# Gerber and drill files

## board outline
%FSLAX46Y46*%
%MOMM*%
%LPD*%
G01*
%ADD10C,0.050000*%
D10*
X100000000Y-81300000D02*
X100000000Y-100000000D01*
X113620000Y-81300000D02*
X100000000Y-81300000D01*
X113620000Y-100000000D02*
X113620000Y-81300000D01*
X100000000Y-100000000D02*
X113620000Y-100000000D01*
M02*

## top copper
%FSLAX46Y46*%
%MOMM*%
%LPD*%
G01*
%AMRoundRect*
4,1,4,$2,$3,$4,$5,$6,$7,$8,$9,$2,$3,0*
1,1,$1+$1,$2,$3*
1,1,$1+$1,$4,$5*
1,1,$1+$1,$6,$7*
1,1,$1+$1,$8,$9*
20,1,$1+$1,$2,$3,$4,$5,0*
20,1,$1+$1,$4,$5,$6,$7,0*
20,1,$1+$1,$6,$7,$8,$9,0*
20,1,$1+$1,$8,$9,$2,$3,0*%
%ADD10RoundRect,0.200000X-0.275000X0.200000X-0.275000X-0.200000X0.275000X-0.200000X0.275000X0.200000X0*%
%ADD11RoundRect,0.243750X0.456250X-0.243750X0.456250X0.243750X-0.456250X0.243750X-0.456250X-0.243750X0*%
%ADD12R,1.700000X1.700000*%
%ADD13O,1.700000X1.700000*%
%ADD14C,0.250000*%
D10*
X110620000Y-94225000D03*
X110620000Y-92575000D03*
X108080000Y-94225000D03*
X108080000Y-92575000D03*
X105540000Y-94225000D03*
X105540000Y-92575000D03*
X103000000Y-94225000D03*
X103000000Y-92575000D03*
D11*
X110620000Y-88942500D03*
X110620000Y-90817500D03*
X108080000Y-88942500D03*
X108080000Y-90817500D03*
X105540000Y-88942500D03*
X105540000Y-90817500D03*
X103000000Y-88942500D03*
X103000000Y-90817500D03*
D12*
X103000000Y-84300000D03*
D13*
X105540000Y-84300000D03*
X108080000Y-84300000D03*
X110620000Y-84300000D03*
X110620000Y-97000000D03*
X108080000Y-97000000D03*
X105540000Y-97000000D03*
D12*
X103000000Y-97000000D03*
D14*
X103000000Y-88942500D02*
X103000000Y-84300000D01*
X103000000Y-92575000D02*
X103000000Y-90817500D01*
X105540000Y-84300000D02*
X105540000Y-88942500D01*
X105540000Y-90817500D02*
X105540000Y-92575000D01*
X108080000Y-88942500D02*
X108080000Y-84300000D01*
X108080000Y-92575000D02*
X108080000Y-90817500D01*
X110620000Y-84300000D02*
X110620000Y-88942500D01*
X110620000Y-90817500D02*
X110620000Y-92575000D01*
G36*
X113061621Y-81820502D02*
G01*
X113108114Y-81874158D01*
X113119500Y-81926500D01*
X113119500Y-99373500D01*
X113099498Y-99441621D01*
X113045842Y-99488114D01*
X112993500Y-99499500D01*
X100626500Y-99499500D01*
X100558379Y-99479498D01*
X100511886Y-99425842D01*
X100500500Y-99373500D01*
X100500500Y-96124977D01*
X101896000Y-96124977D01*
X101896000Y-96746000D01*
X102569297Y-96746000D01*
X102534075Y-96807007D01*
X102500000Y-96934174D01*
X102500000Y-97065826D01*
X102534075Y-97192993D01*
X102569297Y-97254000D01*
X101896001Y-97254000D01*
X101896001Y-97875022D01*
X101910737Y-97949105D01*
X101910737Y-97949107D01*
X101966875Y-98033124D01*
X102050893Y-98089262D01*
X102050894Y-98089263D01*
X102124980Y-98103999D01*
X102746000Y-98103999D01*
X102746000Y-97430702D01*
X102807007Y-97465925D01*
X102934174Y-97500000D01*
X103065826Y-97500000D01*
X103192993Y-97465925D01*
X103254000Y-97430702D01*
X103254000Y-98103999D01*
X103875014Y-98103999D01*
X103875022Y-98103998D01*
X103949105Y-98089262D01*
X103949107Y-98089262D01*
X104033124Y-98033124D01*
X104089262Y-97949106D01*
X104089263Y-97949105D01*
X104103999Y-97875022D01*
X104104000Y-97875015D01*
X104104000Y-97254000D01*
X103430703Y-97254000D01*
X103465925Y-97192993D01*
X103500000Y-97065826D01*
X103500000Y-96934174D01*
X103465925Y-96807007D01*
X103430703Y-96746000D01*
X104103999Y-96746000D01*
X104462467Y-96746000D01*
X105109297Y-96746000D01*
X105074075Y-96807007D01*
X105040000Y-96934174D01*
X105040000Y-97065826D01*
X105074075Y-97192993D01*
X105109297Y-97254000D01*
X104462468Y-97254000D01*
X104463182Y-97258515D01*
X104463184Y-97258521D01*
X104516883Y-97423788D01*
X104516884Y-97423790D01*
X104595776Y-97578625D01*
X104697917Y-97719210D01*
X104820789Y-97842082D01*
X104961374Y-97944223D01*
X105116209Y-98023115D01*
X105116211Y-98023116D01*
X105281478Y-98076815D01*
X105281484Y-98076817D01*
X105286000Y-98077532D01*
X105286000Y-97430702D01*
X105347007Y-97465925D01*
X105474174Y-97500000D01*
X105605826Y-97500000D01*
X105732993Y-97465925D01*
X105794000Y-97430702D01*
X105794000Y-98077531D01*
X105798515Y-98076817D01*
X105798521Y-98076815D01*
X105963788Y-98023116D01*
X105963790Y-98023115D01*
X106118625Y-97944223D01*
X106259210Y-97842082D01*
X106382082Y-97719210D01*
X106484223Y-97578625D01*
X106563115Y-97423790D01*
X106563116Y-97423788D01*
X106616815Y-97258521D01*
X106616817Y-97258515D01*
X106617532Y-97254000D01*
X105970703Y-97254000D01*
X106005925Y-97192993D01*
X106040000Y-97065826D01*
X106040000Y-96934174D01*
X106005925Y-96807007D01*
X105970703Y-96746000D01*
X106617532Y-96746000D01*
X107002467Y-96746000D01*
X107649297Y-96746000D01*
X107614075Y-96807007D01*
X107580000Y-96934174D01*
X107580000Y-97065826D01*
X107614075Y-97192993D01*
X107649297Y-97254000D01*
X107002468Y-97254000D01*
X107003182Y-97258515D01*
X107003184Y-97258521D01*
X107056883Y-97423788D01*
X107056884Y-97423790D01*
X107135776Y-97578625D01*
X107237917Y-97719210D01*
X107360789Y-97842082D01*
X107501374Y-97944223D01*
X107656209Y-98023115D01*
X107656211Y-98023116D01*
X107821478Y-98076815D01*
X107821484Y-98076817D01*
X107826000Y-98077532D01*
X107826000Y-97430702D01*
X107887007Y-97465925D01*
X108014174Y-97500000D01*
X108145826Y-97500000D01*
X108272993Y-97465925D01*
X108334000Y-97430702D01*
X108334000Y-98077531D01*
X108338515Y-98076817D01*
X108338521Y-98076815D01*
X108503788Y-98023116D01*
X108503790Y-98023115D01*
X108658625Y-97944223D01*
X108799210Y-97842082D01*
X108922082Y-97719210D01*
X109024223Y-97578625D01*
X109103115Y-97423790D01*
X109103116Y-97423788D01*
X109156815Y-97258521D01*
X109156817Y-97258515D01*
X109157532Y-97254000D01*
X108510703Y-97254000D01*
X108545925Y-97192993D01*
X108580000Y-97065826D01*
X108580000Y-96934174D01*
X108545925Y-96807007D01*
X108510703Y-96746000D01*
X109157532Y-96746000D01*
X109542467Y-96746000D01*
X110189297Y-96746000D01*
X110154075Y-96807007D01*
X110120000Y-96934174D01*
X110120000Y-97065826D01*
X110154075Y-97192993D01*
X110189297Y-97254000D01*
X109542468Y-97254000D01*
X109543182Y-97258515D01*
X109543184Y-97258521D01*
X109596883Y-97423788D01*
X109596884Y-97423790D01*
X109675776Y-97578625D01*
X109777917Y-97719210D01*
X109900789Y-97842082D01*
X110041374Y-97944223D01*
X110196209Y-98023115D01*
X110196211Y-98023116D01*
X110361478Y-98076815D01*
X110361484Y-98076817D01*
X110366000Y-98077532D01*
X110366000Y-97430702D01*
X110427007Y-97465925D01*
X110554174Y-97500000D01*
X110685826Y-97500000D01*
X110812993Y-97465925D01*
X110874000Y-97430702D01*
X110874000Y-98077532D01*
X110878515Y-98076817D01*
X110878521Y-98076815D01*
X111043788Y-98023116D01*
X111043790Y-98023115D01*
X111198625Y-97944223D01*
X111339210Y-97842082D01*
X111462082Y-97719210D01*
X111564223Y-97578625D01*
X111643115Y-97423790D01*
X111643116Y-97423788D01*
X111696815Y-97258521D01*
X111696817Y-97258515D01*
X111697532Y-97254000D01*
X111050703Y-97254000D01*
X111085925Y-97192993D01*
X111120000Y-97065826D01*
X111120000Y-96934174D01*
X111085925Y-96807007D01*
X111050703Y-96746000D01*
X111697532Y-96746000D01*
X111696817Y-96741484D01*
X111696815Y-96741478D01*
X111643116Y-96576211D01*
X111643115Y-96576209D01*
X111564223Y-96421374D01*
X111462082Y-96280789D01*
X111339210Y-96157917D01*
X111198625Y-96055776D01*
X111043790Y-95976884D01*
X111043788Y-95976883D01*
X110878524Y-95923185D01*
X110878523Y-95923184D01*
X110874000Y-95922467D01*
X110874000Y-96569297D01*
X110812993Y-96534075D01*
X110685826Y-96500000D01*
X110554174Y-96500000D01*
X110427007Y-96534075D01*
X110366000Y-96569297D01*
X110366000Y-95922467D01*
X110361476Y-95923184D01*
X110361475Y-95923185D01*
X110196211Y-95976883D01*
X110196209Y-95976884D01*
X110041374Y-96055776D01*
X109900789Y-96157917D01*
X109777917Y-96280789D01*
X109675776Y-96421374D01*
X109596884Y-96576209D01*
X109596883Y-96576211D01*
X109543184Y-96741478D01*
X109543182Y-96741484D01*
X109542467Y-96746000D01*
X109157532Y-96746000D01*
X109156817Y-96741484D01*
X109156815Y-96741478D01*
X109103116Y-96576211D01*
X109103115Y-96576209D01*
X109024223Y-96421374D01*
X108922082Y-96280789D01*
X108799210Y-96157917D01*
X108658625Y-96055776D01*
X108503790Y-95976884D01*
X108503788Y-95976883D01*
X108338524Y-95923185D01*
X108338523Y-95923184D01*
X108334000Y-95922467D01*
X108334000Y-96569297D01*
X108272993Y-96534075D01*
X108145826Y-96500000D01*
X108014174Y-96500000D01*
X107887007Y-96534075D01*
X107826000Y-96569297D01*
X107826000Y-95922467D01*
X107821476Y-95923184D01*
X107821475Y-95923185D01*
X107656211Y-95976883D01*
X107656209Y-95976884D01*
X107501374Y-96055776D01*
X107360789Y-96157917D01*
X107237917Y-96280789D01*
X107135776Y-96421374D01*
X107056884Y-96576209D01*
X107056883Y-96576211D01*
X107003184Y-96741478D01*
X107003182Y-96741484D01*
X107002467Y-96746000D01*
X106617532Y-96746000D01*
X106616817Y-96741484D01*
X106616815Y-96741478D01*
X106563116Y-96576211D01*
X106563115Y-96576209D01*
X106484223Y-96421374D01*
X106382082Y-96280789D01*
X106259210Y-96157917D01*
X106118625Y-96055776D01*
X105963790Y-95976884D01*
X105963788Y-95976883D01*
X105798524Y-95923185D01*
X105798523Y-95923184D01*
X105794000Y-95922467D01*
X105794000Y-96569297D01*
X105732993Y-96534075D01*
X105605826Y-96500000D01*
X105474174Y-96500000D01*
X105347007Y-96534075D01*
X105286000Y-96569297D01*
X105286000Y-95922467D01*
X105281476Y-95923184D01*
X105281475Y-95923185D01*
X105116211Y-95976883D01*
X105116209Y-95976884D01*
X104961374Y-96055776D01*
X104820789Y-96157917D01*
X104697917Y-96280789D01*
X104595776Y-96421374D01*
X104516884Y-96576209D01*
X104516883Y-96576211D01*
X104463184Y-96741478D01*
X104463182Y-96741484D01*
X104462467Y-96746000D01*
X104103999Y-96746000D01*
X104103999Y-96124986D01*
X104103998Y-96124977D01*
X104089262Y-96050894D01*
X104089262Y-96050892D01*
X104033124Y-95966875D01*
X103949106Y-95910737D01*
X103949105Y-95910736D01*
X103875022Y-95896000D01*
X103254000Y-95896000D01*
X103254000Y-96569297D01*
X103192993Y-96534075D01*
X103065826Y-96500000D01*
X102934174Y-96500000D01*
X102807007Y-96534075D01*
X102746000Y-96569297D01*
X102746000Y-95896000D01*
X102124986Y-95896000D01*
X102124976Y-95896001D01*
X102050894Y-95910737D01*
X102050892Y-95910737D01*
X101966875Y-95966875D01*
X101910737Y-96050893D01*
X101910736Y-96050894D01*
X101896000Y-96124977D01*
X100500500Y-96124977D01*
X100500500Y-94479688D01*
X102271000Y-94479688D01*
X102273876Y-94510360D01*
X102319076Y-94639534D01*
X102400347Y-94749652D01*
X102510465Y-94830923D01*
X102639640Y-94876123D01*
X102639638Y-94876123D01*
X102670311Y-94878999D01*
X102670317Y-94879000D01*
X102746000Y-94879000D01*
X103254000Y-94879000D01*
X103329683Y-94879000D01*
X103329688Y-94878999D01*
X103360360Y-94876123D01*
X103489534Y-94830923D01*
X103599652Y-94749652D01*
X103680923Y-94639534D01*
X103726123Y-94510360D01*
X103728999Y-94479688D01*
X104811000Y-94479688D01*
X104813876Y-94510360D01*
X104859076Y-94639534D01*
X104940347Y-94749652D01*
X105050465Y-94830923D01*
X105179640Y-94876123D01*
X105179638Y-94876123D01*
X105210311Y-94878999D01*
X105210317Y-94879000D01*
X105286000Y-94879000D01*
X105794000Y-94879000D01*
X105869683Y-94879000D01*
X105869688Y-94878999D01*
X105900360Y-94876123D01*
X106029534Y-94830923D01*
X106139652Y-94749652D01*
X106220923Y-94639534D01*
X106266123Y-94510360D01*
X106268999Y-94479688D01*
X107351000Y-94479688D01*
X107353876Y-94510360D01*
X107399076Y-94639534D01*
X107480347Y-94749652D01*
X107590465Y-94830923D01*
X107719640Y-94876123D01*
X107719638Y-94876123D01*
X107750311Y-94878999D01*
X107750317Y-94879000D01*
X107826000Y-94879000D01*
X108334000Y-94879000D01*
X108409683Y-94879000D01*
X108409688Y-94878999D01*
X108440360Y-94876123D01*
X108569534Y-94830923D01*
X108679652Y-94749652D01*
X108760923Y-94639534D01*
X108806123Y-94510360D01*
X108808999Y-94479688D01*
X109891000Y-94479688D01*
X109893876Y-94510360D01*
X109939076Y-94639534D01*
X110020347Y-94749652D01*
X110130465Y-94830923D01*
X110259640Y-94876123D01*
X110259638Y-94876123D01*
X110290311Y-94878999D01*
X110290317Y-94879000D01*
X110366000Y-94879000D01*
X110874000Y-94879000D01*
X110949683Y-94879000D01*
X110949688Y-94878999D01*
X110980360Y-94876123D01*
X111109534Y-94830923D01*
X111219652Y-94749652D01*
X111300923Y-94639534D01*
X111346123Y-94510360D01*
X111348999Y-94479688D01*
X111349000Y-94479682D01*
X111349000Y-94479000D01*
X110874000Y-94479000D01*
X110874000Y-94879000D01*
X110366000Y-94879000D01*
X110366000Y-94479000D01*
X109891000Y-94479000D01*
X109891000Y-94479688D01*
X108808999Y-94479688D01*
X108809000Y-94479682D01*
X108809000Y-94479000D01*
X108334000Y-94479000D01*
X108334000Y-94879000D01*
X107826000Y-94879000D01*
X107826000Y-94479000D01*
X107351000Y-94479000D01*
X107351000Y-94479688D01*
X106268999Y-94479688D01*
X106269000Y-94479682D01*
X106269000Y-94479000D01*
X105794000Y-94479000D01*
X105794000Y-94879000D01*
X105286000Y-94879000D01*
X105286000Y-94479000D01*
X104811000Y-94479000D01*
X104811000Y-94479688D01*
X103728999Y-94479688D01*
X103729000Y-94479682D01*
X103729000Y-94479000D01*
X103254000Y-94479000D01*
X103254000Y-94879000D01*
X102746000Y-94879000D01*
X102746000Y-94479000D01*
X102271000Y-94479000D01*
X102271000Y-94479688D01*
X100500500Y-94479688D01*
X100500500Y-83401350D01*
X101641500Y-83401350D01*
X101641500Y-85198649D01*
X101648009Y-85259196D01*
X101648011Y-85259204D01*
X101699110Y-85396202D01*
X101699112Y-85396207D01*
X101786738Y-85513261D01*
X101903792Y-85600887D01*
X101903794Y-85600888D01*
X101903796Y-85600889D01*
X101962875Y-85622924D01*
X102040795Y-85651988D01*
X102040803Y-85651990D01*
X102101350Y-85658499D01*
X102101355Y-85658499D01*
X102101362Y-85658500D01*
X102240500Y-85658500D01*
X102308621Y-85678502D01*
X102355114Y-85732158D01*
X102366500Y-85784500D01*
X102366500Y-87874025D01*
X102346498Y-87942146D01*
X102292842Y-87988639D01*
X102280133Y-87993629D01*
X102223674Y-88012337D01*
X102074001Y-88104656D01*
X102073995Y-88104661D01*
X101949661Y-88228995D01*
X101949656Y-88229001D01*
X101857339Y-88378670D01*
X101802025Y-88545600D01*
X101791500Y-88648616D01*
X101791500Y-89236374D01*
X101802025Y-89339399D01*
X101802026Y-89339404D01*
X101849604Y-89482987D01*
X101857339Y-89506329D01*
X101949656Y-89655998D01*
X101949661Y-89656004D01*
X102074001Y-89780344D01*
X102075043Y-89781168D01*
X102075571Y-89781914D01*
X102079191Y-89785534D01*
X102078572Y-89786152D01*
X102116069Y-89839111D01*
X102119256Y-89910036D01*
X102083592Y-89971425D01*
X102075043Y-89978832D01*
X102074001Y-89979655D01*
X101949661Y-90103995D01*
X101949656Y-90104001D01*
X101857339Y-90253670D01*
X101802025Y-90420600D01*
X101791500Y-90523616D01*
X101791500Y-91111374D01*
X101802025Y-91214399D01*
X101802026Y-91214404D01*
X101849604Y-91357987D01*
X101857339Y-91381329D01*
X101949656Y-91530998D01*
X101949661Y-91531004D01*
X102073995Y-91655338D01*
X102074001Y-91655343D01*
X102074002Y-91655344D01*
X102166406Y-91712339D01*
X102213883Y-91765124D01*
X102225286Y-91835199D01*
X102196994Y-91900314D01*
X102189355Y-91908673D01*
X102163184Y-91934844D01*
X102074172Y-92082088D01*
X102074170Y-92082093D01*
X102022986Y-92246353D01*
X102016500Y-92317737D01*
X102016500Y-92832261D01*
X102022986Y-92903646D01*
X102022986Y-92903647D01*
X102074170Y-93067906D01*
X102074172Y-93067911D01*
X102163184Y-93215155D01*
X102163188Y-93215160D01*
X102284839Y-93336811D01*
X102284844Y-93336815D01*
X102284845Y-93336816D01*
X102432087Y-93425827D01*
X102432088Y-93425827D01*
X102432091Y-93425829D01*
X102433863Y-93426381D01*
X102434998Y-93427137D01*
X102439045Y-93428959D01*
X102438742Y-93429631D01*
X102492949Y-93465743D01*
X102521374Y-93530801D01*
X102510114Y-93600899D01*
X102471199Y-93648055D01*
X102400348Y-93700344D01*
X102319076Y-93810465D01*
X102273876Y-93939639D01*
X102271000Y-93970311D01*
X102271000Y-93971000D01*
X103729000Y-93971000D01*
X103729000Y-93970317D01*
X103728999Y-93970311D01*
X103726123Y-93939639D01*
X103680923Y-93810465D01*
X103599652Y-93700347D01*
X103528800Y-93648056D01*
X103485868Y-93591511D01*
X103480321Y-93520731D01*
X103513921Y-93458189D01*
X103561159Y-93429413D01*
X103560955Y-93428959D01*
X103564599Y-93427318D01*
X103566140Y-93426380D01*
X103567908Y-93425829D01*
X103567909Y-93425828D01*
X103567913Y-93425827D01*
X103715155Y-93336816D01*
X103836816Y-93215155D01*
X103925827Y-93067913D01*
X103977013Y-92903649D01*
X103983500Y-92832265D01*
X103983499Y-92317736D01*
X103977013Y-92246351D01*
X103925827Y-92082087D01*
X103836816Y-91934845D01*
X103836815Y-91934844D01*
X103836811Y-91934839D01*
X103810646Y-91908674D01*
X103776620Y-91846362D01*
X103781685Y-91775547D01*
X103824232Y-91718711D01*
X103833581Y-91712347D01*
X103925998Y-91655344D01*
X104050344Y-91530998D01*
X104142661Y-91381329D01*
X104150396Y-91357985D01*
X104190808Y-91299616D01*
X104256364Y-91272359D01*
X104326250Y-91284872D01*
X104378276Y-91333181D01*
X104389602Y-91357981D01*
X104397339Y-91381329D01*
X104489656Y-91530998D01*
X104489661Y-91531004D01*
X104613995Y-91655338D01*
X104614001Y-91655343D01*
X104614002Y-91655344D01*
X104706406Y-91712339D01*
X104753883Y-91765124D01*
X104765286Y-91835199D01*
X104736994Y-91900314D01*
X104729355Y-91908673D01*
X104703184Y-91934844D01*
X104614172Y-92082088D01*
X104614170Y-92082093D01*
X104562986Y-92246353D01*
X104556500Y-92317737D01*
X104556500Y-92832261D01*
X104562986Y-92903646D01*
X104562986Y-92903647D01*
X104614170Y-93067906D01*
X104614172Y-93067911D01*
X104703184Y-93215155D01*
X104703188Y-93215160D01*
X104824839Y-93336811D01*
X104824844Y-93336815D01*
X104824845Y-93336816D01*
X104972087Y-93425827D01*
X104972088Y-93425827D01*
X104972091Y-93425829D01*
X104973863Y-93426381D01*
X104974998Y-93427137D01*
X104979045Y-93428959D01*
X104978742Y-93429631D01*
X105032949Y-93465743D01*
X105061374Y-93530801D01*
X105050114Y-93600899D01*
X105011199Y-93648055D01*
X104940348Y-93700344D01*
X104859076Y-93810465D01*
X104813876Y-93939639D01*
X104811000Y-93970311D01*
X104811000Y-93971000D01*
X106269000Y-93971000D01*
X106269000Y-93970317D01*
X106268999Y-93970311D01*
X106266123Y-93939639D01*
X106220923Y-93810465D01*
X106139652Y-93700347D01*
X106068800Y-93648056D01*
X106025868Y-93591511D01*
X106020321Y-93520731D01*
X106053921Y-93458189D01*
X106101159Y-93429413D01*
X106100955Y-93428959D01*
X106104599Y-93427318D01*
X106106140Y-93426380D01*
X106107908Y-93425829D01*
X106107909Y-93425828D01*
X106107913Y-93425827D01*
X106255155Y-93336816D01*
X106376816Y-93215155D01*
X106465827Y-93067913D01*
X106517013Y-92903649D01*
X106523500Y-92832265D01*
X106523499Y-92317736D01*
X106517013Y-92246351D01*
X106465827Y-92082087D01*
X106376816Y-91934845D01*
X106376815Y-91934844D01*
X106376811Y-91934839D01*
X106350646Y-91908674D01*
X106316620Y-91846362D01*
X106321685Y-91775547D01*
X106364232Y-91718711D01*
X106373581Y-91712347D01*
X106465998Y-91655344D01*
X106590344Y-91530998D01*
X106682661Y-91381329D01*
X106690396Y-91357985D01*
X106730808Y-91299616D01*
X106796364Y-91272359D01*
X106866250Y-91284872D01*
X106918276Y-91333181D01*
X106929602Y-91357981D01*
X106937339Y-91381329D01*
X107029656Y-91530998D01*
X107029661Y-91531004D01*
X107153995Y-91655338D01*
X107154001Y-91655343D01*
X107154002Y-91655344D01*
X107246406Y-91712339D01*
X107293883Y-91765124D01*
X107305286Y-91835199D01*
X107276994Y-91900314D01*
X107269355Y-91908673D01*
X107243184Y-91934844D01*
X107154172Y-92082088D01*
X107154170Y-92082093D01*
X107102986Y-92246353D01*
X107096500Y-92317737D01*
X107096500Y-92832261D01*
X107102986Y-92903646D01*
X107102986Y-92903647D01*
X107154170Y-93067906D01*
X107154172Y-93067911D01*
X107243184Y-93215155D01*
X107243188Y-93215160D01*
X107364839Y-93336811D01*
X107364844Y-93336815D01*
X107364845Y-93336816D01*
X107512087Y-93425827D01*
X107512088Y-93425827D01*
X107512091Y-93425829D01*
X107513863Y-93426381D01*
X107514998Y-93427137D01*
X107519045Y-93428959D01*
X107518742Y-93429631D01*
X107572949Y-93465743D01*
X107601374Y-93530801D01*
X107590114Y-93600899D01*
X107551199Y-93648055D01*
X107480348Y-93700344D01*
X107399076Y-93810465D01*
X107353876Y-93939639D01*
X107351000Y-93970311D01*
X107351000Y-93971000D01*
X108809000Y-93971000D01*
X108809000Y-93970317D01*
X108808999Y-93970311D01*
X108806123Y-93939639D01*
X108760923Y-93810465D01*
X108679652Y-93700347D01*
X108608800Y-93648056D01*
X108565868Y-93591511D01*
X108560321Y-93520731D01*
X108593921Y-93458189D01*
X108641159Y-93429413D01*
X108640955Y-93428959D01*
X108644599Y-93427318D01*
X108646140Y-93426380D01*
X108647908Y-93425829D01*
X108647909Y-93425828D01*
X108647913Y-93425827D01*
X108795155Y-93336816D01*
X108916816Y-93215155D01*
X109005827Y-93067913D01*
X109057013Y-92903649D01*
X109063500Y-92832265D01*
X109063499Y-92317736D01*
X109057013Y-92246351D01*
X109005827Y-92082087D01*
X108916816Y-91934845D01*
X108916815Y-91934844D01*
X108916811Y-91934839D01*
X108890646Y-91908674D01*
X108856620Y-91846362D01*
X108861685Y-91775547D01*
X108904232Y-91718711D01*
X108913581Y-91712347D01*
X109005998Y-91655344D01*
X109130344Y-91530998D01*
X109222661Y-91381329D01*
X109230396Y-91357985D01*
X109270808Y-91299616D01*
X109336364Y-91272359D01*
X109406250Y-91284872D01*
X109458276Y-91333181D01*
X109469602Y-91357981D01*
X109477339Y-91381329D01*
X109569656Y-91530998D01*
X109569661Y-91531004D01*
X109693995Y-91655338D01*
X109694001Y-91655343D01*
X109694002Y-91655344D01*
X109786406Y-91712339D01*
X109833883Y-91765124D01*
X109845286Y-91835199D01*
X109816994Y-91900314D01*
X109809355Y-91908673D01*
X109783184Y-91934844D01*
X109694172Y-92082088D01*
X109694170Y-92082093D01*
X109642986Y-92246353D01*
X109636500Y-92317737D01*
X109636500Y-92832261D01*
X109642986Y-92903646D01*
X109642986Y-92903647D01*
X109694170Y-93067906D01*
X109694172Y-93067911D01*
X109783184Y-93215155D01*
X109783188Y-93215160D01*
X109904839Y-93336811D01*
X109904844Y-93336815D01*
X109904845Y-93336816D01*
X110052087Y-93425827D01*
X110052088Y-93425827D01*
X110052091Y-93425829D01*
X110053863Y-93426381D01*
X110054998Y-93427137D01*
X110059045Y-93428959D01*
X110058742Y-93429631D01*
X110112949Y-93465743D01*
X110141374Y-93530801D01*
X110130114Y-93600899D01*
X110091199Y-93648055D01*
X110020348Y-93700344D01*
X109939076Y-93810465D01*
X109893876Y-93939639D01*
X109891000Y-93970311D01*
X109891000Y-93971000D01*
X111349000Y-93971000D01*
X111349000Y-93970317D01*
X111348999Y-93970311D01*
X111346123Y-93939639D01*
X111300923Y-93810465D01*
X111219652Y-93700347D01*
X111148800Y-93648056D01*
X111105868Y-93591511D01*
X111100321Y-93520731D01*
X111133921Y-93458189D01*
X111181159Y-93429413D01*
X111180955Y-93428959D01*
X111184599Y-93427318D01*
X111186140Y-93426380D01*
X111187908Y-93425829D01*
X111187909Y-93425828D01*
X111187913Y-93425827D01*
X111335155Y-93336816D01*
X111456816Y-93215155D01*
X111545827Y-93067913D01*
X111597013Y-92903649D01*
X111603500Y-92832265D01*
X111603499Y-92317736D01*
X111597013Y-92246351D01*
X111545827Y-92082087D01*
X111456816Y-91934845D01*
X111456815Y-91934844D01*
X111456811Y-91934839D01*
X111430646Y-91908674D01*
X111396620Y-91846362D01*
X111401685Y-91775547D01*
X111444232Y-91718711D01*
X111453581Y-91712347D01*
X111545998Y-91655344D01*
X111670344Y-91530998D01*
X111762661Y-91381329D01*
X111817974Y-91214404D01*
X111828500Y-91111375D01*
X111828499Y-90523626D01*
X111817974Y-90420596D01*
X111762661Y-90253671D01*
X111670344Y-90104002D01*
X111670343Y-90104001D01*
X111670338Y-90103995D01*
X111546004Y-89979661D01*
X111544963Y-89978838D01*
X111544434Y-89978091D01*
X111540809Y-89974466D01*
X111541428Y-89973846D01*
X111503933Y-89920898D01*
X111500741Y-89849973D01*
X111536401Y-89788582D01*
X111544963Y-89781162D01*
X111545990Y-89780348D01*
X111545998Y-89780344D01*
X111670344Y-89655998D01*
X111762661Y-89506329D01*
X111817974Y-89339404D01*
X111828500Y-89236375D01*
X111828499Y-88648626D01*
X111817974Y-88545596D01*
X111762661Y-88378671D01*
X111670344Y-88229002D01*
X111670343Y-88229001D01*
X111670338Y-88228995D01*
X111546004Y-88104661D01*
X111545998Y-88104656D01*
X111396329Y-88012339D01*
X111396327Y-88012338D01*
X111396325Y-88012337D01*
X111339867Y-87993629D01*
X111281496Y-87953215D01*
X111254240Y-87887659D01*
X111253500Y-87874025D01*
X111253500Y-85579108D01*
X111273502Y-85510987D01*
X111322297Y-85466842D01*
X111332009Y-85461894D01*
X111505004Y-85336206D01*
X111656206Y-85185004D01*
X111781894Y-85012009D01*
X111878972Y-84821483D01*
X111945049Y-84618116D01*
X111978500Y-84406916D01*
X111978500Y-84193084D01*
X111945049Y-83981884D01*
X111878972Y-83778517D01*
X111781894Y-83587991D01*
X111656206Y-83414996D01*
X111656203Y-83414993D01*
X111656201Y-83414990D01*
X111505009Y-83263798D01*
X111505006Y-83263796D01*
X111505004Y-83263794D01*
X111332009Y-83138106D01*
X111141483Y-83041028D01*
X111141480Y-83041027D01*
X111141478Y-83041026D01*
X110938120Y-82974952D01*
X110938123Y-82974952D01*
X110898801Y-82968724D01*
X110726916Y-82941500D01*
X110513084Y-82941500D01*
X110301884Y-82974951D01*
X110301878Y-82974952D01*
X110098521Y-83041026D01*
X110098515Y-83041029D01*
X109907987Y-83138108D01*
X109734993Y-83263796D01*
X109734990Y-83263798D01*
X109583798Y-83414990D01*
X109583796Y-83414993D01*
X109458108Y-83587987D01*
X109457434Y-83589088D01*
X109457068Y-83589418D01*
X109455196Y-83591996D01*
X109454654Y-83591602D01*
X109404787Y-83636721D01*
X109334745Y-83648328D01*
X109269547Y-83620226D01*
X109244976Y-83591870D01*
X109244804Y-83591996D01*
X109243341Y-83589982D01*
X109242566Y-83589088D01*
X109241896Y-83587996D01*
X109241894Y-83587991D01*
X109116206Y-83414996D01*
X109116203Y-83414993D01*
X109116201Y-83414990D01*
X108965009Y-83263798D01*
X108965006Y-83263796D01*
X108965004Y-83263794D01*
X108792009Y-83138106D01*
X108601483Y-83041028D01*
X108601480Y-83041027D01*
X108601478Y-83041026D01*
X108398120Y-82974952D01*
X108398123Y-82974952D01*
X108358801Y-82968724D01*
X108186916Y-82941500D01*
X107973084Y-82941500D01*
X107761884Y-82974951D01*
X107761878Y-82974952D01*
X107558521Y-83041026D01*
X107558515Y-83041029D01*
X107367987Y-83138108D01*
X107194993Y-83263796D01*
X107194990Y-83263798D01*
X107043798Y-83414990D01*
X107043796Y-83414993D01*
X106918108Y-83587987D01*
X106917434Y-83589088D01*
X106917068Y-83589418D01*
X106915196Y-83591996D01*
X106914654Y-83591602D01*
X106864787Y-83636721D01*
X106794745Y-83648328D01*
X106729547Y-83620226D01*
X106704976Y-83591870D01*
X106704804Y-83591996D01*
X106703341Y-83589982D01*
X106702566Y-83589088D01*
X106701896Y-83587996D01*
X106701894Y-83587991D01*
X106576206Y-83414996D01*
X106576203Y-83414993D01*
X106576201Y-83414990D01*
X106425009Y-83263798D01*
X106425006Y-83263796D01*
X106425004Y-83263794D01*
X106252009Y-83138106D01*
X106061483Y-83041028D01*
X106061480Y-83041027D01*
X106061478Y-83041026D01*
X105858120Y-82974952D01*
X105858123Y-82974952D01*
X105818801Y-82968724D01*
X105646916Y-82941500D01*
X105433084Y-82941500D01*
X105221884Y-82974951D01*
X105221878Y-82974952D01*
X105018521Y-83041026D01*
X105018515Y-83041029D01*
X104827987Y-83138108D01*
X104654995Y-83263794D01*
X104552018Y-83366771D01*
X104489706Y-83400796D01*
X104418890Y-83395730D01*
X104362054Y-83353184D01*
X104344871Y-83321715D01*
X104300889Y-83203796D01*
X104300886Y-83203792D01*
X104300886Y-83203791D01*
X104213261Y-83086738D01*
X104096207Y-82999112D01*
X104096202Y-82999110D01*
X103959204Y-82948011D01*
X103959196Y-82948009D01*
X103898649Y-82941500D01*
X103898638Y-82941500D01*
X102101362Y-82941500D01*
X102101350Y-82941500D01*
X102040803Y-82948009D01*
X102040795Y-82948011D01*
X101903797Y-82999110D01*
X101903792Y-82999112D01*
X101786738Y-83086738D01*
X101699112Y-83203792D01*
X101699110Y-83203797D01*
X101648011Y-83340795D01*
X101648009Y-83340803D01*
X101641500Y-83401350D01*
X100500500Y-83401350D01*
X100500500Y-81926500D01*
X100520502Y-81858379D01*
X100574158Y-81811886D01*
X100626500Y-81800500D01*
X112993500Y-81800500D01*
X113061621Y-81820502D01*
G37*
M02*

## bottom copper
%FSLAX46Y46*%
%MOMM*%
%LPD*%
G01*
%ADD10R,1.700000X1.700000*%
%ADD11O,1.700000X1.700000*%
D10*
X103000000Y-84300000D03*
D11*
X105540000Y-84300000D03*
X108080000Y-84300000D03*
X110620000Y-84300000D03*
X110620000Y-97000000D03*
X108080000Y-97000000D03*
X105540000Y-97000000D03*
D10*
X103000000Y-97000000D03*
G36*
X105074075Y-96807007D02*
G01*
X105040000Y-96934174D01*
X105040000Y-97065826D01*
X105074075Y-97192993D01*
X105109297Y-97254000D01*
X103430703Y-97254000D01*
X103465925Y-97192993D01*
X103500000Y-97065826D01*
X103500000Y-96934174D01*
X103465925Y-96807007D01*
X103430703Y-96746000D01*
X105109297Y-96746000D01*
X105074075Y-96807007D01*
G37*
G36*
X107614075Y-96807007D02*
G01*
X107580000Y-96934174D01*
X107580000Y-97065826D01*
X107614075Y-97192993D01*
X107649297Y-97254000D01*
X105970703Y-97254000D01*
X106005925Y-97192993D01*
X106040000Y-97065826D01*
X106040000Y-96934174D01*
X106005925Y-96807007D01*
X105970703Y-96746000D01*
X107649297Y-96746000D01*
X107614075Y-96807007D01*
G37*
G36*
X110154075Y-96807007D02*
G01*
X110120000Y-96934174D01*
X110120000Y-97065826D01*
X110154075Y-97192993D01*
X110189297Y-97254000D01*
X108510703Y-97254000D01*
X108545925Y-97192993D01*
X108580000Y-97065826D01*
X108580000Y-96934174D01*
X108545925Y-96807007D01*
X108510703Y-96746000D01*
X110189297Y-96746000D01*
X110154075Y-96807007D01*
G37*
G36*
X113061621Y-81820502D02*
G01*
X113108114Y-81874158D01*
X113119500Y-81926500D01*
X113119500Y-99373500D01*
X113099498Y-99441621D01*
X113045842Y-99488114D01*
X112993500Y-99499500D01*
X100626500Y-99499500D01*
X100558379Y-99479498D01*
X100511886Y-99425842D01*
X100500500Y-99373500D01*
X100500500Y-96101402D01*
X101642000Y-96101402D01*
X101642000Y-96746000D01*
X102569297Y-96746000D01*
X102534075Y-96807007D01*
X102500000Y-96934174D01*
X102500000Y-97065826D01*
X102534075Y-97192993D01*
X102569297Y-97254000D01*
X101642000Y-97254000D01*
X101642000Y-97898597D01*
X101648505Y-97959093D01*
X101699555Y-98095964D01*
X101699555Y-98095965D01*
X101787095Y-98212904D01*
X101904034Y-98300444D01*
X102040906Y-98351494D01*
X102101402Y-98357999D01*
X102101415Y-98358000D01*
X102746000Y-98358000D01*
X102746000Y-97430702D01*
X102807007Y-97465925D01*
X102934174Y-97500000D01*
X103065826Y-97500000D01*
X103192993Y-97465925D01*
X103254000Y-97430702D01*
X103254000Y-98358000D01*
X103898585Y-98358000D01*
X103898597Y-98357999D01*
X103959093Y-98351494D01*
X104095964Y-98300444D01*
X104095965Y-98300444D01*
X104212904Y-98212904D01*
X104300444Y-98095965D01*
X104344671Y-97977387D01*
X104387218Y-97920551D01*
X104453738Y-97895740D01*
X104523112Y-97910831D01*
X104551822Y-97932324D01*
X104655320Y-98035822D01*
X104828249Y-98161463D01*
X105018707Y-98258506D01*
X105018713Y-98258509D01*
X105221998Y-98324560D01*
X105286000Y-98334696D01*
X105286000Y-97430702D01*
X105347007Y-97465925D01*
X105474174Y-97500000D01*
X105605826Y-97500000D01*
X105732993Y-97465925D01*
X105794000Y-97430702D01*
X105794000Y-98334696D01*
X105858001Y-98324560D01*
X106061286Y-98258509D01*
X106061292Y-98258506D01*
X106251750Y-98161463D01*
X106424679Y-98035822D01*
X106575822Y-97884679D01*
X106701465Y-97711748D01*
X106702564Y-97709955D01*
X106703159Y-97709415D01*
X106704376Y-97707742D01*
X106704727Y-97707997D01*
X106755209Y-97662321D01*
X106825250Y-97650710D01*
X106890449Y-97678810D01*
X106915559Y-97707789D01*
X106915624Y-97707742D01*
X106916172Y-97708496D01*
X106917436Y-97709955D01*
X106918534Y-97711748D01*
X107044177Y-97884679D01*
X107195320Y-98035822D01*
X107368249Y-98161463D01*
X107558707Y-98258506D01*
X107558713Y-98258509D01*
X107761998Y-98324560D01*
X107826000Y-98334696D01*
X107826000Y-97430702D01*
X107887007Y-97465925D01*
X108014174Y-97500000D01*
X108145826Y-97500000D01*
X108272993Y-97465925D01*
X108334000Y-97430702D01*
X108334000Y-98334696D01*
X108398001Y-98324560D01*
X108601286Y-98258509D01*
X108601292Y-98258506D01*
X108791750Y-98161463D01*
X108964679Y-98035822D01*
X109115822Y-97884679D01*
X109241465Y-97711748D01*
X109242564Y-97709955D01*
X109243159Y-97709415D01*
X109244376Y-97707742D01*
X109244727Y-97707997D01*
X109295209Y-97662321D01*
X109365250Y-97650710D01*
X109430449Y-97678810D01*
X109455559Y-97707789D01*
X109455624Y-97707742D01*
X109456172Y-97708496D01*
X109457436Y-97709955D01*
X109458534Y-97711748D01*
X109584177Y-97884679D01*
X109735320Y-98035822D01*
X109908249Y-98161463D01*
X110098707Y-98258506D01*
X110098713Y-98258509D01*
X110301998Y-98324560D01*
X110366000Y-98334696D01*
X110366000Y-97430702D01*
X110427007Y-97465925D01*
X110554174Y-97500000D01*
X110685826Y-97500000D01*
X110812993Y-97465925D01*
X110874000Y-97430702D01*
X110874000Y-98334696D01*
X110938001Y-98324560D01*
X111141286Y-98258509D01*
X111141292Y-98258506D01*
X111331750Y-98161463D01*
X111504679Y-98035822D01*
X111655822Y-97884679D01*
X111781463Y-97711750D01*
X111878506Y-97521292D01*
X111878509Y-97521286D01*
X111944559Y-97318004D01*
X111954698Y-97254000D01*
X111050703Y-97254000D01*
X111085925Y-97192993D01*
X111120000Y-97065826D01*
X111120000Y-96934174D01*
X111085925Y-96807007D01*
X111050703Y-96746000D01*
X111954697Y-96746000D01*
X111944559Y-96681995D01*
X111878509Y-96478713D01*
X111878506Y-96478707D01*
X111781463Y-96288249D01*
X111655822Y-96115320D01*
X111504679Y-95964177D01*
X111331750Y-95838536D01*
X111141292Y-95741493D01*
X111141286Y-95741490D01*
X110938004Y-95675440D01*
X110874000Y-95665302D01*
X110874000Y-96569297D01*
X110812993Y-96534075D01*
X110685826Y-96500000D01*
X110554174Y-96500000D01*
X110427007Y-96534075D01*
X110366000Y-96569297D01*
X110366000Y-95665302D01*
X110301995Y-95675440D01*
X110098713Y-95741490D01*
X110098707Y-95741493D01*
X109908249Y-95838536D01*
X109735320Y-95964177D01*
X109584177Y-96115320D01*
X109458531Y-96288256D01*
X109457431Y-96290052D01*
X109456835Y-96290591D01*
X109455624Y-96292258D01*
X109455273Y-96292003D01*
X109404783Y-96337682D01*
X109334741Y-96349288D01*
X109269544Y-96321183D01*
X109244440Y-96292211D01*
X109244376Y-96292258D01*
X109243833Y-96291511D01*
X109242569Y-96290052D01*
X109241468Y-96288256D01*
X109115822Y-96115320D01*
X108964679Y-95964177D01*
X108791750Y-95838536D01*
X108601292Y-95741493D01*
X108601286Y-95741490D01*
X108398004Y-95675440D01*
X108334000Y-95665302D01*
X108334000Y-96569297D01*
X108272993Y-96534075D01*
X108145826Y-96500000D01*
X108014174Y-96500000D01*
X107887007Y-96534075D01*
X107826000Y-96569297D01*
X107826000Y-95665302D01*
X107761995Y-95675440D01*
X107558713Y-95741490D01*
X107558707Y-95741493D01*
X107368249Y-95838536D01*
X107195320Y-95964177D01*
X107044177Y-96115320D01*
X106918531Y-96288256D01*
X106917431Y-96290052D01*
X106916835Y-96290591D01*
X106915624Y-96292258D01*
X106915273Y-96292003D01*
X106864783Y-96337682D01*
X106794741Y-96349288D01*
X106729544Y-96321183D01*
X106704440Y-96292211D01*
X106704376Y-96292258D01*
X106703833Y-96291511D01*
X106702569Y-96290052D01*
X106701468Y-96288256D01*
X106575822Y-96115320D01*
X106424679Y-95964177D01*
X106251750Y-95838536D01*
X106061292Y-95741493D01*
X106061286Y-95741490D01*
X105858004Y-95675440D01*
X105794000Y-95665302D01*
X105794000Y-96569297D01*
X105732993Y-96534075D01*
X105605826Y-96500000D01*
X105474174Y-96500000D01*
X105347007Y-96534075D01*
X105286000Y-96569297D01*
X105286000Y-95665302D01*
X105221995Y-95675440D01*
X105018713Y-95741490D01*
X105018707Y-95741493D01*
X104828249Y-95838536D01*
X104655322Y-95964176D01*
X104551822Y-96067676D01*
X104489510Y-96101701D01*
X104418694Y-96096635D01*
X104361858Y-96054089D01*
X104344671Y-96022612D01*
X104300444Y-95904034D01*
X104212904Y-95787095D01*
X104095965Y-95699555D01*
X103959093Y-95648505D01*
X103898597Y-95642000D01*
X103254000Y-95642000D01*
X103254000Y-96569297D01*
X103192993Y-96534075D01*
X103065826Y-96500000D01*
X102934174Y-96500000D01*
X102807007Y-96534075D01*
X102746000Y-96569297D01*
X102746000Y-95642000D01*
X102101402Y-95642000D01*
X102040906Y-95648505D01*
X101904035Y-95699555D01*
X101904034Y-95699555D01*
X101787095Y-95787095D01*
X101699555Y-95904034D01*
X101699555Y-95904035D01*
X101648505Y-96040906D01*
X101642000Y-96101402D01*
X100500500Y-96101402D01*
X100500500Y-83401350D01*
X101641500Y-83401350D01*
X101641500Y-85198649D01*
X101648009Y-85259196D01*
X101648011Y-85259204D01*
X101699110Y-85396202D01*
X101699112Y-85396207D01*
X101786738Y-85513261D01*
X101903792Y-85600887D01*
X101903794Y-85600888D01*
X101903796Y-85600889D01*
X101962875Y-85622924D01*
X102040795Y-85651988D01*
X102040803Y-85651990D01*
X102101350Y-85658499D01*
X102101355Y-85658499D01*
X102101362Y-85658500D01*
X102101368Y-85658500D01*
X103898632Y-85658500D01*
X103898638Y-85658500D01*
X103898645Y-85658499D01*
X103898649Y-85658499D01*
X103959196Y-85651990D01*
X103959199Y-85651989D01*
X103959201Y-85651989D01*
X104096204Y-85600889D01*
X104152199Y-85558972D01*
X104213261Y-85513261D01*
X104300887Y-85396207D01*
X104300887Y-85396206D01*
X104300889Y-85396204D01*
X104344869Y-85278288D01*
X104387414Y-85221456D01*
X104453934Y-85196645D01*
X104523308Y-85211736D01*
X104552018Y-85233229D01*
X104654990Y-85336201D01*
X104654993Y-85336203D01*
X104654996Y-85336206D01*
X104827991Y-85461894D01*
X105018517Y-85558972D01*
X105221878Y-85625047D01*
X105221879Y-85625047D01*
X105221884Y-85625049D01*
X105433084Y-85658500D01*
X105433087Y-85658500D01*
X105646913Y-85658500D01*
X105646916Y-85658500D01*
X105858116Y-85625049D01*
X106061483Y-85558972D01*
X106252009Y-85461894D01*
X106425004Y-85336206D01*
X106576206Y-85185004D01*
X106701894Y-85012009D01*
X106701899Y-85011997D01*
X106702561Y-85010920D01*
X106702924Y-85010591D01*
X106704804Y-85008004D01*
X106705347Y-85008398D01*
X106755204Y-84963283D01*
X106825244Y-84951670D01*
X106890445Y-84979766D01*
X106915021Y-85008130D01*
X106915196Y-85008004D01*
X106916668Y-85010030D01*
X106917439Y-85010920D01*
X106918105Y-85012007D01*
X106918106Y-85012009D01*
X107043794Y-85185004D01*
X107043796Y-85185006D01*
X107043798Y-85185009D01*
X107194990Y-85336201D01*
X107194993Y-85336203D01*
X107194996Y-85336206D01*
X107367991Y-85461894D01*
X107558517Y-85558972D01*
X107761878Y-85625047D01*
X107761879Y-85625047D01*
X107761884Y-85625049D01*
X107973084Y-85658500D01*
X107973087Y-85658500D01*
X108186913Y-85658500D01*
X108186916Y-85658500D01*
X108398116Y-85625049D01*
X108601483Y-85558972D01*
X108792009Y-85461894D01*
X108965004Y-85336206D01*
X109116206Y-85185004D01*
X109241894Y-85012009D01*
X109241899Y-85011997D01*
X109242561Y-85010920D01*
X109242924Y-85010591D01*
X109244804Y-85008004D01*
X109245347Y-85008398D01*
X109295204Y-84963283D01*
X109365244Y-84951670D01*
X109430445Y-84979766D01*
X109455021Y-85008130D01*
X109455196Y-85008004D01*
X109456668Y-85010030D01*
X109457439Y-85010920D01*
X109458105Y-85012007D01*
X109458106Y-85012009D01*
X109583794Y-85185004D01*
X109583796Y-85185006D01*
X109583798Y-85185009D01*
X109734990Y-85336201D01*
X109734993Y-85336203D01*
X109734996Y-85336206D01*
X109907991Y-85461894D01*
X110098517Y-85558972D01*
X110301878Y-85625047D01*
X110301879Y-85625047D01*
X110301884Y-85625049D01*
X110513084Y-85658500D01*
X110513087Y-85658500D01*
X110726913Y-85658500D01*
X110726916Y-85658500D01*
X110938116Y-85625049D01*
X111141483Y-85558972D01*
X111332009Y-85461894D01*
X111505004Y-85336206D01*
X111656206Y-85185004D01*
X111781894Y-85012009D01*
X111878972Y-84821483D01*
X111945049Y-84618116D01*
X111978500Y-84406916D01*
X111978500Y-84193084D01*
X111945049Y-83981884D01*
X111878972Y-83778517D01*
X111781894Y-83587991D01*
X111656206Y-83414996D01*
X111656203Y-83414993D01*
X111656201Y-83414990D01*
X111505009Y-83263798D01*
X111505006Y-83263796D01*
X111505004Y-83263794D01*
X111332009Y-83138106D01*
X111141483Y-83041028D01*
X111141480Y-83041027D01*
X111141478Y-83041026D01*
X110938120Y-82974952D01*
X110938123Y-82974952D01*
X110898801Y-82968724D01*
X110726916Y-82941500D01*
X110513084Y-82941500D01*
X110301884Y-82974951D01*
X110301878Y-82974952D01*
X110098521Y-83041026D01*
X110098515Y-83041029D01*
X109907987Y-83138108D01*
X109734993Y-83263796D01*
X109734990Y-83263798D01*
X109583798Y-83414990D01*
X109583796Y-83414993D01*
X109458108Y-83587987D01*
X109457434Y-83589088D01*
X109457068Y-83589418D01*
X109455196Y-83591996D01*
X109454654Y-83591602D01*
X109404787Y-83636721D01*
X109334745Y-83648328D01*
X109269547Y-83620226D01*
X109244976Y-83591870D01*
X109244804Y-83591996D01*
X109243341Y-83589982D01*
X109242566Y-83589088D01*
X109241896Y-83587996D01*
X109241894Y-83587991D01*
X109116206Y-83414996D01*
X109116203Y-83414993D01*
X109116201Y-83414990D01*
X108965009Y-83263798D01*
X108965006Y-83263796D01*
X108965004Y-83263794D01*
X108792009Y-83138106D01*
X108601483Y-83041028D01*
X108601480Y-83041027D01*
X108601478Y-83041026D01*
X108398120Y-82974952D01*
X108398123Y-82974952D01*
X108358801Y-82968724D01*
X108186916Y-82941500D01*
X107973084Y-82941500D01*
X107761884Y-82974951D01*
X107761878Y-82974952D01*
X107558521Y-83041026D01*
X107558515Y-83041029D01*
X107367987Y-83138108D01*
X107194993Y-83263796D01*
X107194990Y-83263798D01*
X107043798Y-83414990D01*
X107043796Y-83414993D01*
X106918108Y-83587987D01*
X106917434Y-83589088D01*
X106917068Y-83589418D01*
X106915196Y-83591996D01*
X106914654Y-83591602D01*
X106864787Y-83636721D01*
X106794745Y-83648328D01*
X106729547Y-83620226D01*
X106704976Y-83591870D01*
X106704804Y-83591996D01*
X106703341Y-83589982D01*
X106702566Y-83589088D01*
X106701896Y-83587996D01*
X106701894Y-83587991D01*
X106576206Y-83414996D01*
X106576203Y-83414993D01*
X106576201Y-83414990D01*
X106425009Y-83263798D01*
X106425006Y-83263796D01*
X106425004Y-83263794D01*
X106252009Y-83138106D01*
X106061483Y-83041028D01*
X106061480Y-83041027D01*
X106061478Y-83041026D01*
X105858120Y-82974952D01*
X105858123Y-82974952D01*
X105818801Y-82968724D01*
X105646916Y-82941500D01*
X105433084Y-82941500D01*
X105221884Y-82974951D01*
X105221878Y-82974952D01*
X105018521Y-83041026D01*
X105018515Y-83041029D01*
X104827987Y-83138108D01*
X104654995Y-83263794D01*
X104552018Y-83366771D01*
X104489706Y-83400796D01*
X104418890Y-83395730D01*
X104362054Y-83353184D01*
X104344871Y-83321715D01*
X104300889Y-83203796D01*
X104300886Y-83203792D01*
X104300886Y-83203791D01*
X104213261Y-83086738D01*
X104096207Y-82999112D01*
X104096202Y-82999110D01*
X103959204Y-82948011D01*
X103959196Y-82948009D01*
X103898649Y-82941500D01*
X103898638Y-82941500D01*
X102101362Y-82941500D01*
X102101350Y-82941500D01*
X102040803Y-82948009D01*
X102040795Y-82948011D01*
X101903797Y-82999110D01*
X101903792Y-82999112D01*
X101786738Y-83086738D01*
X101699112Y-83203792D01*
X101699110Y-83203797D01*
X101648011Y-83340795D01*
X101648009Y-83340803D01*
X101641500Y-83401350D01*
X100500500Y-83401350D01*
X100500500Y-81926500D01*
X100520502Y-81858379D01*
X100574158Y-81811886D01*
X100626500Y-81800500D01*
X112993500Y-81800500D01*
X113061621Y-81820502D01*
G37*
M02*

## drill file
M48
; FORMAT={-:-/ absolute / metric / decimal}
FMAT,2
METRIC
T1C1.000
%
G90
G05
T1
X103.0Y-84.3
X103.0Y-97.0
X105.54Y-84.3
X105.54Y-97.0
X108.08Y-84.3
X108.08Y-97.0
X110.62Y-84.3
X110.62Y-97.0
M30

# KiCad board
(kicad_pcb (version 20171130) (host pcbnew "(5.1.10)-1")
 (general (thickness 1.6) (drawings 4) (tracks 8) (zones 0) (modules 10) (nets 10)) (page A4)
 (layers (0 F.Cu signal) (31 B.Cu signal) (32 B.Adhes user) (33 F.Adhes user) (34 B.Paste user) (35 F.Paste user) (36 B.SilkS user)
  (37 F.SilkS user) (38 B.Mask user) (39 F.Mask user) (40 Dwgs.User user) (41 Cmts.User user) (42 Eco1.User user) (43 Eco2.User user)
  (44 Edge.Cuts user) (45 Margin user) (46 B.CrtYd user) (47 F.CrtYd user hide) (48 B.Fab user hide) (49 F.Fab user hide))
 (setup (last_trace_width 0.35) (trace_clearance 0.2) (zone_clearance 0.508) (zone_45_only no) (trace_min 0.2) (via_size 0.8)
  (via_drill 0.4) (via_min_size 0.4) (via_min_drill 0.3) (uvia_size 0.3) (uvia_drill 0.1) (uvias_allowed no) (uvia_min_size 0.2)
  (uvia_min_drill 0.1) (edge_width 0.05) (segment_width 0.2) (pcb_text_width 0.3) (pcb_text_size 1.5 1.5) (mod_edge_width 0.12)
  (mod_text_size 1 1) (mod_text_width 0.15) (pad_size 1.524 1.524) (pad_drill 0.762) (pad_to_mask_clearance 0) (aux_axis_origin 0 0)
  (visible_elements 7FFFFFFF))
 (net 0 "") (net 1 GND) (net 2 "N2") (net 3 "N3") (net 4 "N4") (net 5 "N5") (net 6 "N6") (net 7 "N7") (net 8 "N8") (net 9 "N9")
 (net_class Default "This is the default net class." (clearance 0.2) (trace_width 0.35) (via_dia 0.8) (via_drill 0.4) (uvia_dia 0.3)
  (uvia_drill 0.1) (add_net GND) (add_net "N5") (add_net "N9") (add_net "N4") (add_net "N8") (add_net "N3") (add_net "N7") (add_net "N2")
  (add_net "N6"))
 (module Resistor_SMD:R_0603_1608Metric (layer F.Cu) (at 110.62 93.4 270)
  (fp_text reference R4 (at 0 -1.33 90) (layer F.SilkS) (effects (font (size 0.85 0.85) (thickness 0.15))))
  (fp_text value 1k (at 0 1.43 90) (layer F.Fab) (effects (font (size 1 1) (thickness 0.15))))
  (pad 2 smd roundrect (at 0.825 0 270) (size 0.8 0.95) (layers F.Cu F.Paste F.Mask) (roundrect_rratio 0.25) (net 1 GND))
  (pad 1 smd roundrect (at -0.825 0 270) (size 0.8 0.95) (layers F.Cu F.Paste F.Mask) (roundrect_rratio 0.25) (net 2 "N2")))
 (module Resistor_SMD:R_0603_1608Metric (layer F.Cu) (at 108.08 93.4 270)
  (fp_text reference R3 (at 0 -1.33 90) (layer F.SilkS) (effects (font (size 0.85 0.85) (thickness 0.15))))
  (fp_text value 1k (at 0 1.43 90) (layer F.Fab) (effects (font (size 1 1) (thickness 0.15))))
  (pad 2 smd roundrect (at 0.825 0 270) (size 0.8 0.95) (layers F.Cu F.Paste F.Mask) (roundrect_rratio 0.25) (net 1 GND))
  (pad 1 smd roundrect (at -0.825 0 270) (size 0.8 0.95) (layers F.Cu F.Paste F.Mask) (roundrect_rratio 0.25) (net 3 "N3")))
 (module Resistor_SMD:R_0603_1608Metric (layer F.Cu) (at 105.54 93.4 270)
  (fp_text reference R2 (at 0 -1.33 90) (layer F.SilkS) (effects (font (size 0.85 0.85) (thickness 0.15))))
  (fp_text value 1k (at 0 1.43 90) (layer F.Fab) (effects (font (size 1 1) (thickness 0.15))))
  (pad 2 smd roundrect (at 0.825 0 270) (size 0.8 0.95) (layers F.Cu F.Paste F.Mask) (roundrect_rratio 0.25) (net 1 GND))
  (pad 1 smd roundrect (at -0.825 0 270) (size 0.8 0.95) (layers F.Cu F.Paste F.Mask) (roundrect_rratio 0.25) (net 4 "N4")))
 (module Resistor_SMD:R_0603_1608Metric (layer F.Cu) (at 103 93.4 270)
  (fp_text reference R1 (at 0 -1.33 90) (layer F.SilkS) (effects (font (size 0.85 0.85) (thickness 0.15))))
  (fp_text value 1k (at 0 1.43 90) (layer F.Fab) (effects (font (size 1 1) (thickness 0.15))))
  (pad 2 smd roundrect (at 0.825 0 270) (size 0.8 0.95) (layers F.Cu F.Paste F.Mask) (roundrect_rratio 0.25) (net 1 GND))
  (pad 1 smd roundrect (at -0.825 0 270) (size 0.8 0.95) (layers F.Cu F.Paste F.Mask) (roundrect_rratio 0.25) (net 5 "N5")))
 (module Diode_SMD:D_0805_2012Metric (layer F.Cu) (at 110.62 89.88 90)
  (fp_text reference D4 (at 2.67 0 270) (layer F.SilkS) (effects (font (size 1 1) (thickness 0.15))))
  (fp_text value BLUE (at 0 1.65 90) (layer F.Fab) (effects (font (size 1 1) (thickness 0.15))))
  (pad 2 smd roundrect (at 0.9375 0 90) (size 0.975 1.4) (layers F.Cu F.Paste F.Mask) (roundrect_rratio 0.25) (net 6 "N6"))
  (pad 1 smd roundrect (at -0.9375 0 90) (size 0.975 1.4) (layers F.Cu F.Paste F.Mask) (roundrect_rratio 0.25) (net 2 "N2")))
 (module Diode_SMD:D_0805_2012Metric (layer F.Cu) (at 108.08 89.88 90)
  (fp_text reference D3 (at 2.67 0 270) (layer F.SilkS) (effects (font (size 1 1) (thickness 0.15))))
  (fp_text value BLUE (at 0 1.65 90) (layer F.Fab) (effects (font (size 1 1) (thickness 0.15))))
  (pad 2 smd roundrect (at 0.9375 0 90) (size 0.975 1.4) (layers F.Cu F.Paste F.Mask) (roundrect_rratio 0.25) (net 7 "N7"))
  (pad 1 smd roundrect (at -0.9375 0 90) (size 0.975 1.4) (layers F.Cu F.Paste F.Mask) (roundrect_rratio 0.25) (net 3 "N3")))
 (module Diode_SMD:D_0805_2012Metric (layer F.Cu) (at 105.54 89.88 90)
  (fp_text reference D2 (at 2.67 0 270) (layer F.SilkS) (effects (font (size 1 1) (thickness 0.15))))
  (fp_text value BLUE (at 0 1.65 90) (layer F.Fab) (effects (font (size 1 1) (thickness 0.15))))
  (pad 2 smd roundrect (at 0.9375 0 90) (size 0.975 1.4) (layers F.Cu F.Paste F.Mask) (roundrect_rratio 0.25) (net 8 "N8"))
  (pad 1 smd roundrect (at -0.9375 0 90) (size 0.975 1.4) (layers F.Cu F.Paste F.Mask) (roundrect_rratio 0.25) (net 4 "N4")))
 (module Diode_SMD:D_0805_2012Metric (layer F.Cu) (at 103 89.88 90)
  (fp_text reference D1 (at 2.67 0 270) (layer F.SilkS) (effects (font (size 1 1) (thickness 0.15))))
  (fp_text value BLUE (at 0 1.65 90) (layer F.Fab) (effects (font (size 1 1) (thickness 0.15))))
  (pad 2 smd roundrect (at 0.9375 0 90) (size 0.975 1.4) (layers F.Cu F.Paste F.Mask) (roundrect_rratio 0.25) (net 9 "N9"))
  (pad 1 smd roundrect (at -0.9375 0 90) (size 0.975 1.4) (layers F.Cu F.Paste F.Mask) (roundrect_rratio 0.25) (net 5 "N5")))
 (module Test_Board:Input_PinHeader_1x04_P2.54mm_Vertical (layer B.Cu) (at 103 84.3 270)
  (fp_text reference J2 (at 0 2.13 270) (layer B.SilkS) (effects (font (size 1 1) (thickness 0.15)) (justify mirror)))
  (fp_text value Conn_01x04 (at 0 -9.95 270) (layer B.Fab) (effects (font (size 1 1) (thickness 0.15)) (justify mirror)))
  (pad 1 thru_hole rect (at 0 0 270) (size 1.7 1.7) (drill 1) (layers *.Cu *.Mask) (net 9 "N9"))
  (pad 2 thru_hole oval (at 0 -2.54 270) (size 1.7 1.7) (drill 1) (layers *.Cu *.Mask) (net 8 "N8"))
  (pad 3 thru_hole oval (at 0 -5.08 270) (size 1.7 1.7) (drill 1) (layers *.Cu *.Mask) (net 7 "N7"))
  (pad 4 thru_hole oval (at 0 -7.62 270) (size 1.7 1.7) (drill 1) (layers *.Cu *.Mask) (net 6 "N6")))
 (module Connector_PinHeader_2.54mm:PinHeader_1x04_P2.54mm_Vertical (layer B.Cu) (at 103 97 270)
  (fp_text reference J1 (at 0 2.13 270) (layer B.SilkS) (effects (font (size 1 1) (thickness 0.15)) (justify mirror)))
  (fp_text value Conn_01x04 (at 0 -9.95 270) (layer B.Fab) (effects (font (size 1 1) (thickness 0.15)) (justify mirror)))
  (pad 4 thru_hole oval (at 0 -7.62 270) (size 1.7 1.7) (drill 1) (layers *.Cu *.Mask) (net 1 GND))
  (pad 3 thru_hole oval (at 0 -5.08 270) (size 1.7 1.7) (drill 1) (layers *.Cu *.Mask) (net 1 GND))
  (pad 2 thru_hole oval (at 0 -2.54 270) (size 1.7 1.7) (drill 1) (layers *.Cu *.Mask) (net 1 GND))
  (pad 1 thru_hole rect (at 0 0 270) (size 1.7 1.7) (drill 1) (layers *.Cu *.Mask) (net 1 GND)))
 (gr_line (start 100 81.3) (end 100 100) (layer Edge.Cuts) (width 0.05))
 (gr_line (start 113.62 81.3) (end 100 81.3) (layer Edge.Cuts) (width 0.05))
 (gr_line (start 113.62 100) (end 113.62 81.3) (layer Edge.Cuts) (width 0.05))
 (gr_line (start 100 100) (end 113.62 100) (layer Edge.Cuts) (width 0.05))
 (segment (start 103 88.9425) (end 103 84.3) (width 0.25) (layer F.Cu) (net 9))
 (segment (start 103 92.575) (end 103 90.8175) (width 0.25) (layer F.Cu) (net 5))
 (segment (start 105.54 84.3) (end 105.54 88.9425) (width 0.25) (layer F.Cu) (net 8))
 (segment (start 105.54 90.8175) (end 105.54 92.575) (width 0.25) (layer F.Cu) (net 4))
 (segment (start 108.08 88.9425) (end 108.08 84.3) (width 0.25) (layer F.Cu) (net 7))
 (segment (start 108.08 92.575) (end 108.08 90.8175) (width 0.25) (layer F.Cu) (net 3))
 (segment (start 110.62 84.3) (end 110.62 88.9425) (width 0.25) (layer F.Cu) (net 6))
 (segment (start 110.62 90.8175) (end 110.62 92.575) (width 0.25) (layer F.Cu) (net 2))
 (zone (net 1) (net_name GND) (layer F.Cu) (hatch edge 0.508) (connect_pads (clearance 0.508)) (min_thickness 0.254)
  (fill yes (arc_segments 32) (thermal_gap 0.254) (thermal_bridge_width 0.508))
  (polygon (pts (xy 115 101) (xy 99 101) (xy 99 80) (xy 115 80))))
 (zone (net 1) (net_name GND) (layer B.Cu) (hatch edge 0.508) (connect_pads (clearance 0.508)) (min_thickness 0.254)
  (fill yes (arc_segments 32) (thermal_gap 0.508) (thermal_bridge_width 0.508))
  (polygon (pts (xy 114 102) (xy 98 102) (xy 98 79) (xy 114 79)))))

